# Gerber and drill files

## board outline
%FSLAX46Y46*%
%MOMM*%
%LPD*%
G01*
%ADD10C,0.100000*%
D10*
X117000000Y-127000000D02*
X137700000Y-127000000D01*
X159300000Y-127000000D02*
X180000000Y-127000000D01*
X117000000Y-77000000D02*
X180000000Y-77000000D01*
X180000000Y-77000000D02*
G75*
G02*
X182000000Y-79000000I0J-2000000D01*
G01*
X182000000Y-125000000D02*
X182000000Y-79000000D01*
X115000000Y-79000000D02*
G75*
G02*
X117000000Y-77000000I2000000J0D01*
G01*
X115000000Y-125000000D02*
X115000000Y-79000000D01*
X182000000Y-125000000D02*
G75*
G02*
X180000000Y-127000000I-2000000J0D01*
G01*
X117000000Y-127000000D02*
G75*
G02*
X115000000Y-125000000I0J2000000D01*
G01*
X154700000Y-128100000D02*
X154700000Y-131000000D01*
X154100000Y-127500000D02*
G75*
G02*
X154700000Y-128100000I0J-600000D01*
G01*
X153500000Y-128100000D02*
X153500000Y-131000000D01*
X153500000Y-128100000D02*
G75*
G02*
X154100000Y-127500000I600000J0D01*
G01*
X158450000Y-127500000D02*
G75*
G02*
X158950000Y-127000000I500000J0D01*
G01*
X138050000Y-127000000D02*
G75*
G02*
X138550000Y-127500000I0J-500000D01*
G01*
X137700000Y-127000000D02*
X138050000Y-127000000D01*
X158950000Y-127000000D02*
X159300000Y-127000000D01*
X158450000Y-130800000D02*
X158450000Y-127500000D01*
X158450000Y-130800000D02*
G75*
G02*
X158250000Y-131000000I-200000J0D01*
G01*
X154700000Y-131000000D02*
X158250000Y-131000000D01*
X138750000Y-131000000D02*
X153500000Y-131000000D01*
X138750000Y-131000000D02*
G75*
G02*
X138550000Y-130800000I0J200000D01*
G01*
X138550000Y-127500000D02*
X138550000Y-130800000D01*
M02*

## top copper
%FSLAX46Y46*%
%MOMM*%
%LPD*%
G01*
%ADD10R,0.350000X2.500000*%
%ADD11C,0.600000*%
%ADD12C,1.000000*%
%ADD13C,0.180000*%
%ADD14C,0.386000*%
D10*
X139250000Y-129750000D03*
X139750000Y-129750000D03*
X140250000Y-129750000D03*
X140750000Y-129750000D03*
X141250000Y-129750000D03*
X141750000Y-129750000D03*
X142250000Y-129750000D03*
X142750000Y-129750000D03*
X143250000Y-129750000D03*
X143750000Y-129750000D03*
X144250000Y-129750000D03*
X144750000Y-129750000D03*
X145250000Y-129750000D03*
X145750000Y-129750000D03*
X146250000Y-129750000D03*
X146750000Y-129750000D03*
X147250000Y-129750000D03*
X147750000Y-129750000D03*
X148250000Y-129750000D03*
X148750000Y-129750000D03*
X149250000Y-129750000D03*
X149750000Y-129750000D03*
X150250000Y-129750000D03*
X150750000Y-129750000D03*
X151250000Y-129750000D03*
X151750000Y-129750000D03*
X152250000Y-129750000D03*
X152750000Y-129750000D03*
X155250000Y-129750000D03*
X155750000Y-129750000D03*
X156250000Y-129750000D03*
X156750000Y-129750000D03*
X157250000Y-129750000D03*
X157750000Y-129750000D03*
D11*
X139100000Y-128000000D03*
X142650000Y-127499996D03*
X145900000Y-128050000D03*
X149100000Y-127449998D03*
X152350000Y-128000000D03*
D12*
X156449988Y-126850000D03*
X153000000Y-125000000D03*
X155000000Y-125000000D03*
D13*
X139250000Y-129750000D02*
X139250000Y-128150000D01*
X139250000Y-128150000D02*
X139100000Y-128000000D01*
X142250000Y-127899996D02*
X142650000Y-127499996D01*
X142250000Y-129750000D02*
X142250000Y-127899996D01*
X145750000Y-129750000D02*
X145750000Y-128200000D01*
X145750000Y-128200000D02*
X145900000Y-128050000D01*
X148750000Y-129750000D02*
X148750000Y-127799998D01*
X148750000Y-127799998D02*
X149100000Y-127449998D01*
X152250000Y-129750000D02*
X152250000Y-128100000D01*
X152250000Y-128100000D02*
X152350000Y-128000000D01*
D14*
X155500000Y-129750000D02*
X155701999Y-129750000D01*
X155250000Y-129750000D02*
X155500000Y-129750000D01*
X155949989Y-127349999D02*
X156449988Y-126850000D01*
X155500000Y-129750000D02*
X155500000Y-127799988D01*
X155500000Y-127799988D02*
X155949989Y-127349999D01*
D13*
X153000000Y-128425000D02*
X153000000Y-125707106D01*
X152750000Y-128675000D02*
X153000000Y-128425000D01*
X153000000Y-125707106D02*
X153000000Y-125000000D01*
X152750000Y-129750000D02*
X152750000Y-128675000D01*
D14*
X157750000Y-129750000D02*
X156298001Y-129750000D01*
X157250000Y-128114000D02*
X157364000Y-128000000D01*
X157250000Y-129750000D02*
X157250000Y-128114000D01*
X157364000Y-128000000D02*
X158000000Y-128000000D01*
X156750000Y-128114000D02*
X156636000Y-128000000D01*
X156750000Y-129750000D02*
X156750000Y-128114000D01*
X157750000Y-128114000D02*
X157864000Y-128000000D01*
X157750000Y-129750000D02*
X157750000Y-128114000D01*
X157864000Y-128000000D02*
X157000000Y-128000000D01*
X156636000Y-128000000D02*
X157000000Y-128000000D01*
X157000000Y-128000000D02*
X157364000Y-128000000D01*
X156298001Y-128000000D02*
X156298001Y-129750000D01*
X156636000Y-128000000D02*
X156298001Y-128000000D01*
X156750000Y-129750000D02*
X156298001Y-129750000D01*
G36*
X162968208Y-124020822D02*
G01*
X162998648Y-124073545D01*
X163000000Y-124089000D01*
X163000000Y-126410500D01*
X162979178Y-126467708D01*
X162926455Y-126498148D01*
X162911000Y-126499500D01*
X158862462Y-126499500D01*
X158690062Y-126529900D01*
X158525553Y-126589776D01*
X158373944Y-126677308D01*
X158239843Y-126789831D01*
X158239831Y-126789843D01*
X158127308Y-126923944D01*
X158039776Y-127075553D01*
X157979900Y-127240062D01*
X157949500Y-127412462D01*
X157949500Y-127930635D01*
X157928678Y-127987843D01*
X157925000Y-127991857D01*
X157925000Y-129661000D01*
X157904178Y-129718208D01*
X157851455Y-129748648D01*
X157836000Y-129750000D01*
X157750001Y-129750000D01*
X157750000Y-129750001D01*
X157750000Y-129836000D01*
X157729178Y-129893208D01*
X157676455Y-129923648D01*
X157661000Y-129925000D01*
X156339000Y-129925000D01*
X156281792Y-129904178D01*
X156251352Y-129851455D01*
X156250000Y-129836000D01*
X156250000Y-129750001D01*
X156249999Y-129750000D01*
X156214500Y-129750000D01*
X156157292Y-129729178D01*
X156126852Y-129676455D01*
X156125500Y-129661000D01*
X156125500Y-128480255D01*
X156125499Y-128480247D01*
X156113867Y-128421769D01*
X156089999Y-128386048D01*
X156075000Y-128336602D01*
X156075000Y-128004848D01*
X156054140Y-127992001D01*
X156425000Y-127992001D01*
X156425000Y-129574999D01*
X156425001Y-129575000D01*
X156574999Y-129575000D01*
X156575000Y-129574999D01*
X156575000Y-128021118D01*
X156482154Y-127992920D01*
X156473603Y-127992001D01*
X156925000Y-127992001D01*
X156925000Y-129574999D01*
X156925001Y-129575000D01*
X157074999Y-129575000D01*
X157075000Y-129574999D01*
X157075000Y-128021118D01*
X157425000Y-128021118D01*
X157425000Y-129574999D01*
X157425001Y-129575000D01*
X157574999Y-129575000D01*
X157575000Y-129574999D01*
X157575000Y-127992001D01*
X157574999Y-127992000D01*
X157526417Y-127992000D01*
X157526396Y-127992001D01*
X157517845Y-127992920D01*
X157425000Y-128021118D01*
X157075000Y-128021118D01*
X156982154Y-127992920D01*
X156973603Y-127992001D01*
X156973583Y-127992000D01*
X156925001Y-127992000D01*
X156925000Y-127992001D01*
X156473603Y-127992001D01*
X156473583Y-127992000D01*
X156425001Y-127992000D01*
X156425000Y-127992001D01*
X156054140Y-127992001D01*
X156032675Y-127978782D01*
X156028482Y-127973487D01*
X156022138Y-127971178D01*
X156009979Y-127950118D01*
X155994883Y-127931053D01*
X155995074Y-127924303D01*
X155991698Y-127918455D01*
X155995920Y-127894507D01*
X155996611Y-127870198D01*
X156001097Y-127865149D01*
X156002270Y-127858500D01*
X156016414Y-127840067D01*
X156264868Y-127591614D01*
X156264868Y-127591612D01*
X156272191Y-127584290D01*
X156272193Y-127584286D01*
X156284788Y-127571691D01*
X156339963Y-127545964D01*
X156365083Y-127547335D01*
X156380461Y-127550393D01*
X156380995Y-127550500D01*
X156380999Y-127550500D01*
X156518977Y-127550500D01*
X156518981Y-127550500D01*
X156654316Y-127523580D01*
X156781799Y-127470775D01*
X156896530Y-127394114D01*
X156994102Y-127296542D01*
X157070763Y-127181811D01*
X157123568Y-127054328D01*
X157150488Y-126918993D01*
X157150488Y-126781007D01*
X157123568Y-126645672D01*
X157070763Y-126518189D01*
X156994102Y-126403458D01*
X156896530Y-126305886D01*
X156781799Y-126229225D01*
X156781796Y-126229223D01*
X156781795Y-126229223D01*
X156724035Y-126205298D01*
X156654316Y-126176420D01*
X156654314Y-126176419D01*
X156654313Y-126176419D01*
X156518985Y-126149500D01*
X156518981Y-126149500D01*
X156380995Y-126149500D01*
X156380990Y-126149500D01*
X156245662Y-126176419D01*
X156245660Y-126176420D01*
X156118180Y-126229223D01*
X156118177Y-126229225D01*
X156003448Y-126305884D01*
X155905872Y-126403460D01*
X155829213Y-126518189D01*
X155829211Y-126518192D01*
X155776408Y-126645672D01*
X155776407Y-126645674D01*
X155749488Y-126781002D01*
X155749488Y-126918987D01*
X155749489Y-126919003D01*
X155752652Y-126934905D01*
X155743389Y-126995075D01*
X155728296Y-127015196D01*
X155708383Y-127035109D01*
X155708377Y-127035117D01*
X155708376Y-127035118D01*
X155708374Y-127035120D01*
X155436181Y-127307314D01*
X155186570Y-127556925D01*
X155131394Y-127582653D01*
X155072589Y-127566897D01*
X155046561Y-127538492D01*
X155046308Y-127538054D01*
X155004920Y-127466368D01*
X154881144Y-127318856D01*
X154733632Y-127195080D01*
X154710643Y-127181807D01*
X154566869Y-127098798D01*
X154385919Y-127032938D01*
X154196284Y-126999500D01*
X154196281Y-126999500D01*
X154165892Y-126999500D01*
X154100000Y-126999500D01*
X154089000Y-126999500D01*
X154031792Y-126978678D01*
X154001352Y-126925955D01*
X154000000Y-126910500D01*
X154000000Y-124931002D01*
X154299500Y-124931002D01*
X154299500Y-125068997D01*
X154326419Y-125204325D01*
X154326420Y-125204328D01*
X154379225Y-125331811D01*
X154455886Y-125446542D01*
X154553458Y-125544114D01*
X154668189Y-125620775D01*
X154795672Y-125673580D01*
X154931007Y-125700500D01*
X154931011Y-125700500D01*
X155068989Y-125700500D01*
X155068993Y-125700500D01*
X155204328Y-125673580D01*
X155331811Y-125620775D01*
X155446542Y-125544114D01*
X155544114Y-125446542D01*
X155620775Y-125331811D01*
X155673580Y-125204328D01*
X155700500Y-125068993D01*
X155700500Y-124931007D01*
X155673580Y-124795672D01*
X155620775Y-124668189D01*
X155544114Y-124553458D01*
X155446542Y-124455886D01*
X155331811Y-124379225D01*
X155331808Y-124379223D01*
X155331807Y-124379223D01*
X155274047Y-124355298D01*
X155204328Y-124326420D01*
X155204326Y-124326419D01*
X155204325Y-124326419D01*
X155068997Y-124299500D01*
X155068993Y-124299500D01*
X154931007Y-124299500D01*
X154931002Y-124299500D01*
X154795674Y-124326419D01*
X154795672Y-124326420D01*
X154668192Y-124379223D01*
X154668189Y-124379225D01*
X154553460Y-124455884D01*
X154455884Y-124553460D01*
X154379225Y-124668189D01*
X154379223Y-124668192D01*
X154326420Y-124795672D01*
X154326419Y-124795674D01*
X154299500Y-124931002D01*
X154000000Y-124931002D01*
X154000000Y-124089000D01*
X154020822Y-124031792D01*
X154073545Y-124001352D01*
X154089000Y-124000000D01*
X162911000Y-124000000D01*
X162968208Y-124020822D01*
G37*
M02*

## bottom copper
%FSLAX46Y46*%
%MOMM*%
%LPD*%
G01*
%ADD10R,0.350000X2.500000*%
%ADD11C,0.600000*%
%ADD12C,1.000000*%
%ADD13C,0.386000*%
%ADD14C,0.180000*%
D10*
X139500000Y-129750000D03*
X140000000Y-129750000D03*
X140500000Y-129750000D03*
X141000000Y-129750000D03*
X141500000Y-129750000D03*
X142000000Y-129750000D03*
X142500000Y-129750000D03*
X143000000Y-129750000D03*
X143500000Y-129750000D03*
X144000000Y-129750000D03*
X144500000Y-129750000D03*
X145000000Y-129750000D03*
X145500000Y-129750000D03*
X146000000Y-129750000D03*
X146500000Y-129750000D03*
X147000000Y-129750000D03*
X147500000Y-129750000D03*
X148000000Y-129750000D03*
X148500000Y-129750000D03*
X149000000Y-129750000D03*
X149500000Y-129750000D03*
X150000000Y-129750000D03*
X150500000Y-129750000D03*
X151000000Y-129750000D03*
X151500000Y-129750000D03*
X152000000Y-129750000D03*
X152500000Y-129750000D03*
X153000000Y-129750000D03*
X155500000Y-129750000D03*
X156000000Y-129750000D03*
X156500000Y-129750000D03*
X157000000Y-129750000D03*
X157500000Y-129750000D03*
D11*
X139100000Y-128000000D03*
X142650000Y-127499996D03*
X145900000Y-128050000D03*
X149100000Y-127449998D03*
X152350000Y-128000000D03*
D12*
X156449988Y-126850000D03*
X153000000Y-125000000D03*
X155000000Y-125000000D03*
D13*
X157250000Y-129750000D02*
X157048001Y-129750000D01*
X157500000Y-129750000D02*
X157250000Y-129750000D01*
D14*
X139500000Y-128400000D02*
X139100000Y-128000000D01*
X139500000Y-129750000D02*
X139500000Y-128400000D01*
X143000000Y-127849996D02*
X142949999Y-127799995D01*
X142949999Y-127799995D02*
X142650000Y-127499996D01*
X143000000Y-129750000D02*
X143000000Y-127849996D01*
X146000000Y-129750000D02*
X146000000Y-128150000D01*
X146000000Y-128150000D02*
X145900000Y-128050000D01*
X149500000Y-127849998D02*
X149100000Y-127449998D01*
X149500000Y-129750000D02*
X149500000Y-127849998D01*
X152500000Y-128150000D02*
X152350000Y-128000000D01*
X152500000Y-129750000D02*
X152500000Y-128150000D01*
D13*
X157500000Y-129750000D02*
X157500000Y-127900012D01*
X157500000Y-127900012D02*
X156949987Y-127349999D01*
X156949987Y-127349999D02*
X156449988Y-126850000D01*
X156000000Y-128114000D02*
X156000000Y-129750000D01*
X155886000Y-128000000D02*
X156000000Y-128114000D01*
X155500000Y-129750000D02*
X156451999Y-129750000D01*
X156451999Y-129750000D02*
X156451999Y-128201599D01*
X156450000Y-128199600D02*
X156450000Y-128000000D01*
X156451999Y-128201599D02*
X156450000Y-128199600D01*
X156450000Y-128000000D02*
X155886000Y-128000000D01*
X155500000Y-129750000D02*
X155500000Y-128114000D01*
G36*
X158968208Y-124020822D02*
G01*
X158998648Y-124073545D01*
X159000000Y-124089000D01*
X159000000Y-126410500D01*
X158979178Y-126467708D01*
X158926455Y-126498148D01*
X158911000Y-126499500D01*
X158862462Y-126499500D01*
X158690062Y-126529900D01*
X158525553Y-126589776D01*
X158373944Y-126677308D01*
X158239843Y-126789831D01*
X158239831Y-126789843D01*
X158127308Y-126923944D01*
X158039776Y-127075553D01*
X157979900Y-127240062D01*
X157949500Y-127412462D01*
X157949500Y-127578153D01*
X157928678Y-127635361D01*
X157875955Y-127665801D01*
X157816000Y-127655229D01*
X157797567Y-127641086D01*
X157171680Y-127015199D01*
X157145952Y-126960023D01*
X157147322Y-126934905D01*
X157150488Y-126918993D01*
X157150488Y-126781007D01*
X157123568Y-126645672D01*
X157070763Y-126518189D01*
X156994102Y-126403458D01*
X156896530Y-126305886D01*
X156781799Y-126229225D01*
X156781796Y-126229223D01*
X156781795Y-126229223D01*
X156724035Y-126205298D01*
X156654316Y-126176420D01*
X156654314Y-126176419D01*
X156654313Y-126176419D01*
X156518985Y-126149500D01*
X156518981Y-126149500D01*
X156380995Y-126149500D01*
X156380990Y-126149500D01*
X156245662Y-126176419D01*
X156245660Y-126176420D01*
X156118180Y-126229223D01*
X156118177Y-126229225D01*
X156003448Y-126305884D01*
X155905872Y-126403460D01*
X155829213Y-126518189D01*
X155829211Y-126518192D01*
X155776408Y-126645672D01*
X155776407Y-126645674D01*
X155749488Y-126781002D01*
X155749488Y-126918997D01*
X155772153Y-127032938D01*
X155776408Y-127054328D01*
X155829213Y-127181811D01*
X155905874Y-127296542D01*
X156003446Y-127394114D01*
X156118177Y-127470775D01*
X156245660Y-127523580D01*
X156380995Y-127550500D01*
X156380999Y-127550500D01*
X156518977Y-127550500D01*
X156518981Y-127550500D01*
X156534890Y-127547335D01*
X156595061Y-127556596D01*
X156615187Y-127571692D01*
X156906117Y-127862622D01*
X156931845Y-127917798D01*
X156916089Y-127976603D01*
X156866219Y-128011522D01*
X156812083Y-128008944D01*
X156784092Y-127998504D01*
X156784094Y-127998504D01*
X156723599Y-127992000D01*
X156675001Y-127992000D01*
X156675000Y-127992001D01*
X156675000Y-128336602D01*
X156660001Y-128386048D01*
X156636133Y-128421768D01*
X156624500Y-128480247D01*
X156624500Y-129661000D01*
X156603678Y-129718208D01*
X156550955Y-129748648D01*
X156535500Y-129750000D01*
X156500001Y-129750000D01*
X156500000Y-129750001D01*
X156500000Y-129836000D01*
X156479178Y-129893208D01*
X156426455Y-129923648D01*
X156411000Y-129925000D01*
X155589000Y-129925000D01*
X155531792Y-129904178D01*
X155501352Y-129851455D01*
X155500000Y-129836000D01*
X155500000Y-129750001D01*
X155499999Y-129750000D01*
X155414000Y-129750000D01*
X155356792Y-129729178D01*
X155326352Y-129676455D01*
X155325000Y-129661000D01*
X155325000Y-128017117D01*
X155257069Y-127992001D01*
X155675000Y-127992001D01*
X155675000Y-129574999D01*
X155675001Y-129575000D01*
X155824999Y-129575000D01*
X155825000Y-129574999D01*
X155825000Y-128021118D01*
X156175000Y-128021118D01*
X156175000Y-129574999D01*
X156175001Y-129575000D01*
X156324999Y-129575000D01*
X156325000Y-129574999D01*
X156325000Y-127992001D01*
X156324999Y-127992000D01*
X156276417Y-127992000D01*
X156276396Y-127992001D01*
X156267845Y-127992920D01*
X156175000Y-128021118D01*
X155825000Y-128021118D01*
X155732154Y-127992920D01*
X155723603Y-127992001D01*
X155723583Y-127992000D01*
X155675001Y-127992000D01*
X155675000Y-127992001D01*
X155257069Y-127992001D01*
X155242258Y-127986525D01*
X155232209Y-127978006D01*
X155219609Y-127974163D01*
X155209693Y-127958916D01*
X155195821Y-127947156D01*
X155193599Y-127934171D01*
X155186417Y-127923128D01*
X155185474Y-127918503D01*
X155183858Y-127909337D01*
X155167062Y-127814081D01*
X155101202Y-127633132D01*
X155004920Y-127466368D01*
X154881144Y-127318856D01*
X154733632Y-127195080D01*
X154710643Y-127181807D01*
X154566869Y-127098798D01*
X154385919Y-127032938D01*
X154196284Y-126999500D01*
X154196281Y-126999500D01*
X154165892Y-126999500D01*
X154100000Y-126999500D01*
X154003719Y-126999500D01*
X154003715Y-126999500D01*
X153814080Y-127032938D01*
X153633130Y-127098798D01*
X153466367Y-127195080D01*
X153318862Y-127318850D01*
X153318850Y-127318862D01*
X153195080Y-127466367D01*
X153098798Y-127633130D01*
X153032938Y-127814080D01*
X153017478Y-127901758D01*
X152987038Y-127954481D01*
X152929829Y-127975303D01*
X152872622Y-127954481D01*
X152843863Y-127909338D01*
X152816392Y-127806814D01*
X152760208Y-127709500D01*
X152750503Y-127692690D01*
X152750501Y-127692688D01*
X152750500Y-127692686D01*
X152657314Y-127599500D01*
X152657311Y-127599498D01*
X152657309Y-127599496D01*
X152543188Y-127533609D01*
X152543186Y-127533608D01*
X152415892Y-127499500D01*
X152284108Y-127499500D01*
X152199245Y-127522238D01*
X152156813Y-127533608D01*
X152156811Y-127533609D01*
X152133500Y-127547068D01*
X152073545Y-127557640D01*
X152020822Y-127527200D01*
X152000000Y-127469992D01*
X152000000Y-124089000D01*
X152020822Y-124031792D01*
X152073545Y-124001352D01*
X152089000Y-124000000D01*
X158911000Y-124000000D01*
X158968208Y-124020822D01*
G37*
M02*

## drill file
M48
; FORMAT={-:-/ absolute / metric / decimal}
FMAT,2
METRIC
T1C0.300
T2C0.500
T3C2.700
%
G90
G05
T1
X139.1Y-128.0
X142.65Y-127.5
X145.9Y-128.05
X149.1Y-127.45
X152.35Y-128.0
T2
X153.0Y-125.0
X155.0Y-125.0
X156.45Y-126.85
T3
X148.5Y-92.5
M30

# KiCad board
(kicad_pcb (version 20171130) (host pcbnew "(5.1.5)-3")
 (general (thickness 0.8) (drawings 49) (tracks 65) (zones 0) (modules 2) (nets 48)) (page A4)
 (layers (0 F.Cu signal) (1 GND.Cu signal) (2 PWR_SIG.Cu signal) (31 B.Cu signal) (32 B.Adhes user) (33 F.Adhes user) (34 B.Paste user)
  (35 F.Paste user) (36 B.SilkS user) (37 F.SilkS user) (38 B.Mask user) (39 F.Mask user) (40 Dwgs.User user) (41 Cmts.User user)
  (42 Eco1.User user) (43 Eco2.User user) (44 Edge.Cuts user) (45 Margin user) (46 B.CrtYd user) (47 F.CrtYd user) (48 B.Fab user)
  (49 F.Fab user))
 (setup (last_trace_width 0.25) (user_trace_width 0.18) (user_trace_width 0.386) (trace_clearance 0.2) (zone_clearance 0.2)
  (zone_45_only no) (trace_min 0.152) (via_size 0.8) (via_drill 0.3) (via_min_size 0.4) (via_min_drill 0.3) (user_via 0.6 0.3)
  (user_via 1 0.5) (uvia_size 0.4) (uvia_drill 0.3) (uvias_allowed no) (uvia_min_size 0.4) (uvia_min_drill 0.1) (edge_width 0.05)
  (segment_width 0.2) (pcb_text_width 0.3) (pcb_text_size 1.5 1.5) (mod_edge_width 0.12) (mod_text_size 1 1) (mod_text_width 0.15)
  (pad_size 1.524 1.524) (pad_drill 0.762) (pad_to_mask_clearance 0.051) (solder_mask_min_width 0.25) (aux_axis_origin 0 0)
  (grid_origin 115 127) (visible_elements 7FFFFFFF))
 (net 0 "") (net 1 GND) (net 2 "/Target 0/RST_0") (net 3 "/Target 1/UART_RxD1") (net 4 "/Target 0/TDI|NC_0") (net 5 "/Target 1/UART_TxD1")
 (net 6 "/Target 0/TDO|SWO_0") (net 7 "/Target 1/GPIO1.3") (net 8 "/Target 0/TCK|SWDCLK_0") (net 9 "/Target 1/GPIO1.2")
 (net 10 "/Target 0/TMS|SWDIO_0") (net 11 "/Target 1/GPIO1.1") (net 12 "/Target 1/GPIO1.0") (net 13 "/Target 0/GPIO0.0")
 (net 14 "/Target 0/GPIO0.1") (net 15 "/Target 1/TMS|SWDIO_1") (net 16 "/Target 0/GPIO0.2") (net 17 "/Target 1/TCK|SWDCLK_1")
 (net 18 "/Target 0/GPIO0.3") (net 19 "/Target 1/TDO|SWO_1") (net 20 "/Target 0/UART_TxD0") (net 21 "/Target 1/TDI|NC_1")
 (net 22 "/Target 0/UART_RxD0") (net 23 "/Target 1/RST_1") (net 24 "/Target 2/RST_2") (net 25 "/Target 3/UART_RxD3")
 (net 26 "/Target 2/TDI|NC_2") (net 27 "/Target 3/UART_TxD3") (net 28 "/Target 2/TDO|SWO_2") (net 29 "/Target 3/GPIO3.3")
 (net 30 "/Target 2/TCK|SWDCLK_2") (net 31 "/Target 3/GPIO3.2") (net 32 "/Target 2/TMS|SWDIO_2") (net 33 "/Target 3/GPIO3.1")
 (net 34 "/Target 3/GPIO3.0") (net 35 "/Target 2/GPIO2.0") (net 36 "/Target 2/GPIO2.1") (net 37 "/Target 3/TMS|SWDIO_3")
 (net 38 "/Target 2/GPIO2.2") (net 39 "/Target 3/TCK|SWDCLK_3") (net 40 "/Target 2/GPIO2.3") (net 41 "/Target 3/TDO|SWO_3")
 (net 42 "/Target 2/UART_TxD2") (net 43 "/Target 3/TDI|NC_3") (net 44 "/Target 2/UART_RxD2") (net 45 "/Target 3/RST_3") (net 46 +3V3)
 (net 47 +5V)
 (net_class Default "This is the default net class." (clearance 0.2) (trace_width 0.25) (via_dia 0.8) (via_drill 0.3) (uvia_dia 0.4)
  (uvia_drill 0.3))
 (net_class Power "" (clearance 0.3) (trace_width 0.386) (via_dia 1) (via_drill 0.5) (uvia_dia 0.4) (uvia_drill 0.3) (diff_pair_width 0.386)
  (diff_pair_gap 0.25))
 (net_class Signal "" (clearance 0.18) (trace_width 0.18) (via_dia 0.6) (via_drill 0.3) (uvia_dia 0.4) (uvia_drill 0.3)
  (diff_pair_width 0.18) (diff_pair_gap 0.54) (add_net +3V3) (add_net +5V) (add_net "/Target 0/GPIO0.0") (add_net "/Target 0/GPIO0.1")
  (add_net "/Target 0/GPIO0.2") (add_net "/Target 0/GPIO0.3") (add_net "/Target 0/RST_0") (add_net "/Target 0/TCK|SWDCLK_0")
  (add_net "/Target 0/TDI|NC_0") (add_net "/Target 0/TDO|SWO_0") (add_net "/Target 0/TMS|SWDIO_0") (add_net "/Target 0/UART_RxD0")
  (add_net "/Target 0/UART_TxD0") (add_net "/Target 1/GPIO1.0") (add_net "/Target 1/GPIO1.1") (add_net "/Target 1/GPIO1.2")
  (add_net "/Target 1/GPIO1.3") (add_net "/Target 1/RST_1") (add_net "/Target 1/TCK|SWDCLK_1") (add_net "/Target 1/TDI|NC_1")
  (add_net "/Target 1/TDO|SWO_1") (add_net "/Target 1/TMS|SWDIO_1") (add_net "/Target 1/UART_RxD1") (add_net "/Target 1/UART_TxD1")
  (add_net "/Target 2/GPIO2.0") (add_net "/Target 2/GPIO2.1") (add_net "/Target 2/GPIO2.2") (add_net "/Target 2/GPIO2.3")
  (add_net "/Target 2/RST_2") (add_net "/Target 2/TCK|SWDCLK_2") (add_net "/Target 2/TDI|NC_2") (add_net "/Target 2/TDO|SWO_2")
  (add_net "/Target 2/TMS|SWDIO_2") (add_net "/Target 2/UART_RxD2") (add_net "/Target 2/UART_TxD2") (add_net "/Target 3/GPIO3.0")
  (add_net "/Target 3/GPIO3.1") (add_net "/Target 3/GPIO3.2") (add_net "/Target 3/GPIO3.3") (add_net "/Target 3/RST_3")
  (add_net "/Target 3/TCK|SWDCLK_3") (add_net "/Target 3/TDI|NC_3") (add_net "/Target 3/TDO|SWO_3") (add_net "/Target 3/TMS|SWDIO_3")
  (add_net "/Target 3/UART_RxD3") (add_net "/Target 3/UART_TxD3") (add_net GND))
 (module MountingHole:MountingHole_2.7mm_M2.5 (layer F.Cu) (at 148.5 92.5)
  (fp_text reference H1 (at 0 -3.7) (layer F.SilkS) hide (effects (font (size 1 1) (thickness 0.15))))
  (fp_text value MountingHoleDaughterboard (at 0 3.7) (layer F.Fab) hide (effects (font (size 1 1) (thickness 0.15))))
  (pad 1 np_thru_hole circle (at 0 0) (size 2.7 2.7) (drill 2.7) (layers *.Cu *.Mask)))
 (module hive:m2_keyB (layer F.Cu) (at 148.5 131)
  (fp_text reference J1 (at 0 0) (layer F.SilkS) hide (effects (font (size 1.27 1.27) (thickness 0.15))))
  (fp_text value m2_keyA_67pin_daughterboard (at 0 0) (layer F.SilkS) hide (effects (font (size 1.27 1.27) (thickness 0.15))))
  (fp_line (start 6.2 -2.9) (end 6.2 0) (layer Edge.Cuts) (width 0.1))
  (fp_arc (start 5.6 -2.9) (end 5.6 -3.5) (angle 90) (layer Edge.Cuts) (width 0.1))
  (fp_line (start 5 -2.9) (end 5 0) (layer Edge.Cuts) (width 0.1))
  (fp_arc (start 5.6 -2.9) (end 5.6 -3.5) (angle -90) (layer Edge.Cuts) (width 0.1))
  (fp_arc (start 10.45 -3.5) (end 9.95 -3.5) (angle 90) (layer Edge.Cuts) (width 0.1))
  (fp_arc (start -10.45 -3.5) (end -10.45 -4) (angle 90) (layer Edge.Cuts) (width 0.1))
  (fp_line (start -10.8 -4) (end -10.45 -4) (layer Edge.Cuts) (width 0.1))
  (fp_line (start 10.45 -4) (end 10.8 -4) (layer Edge.Cuts) (width 0.1))
  (fp_line (start 9.95 -0.2) (end 9.95 -3.5) (layer Edge.Cuts) (width 0.1))
  (fp_arc (start 9.75 -0.2) (end 9.75 0) (angle -90) (layer Edge.Cuts) (width 0.1))
  (fp_line (start 6.2 0) (end 9.75 0) (layer Edge.Cuts) (width 0.1))
  (fp_line (start -9.75 0) (end 5 0) (layer Edge.Cuts) (width 0.1))
  (fp_arc (start -9.75 -0.2) (end -9.95 -0.2) (angle -90) (layer Edge.Cuts) (width 0.1))
  (fp_line (start -9.95 -3.5) (end -9.95 -0.2) (layer Edge.Cuts) (width 0.1))
  (pad 75 smd rect (at -9.25 -1.25) (size 0.35 2.5) (layers F.Cu F.Paste F.Mask) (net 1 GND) (solder_mask_margin 0.1016))
  (pad 74 smd rect (at -9 -1.25) (size 0.35 2.5) (layers B.Cu B.Paste B.Mask) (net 1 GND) (solder_mask_margin 0.1016))
  (pad 73 smd rect (at -8.75 -1.25) (size 0.35 2.5) (layers F.Cu F.Paste F.Mask) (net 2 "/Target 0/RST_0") (solder_mask_margin 0.1016))
  (pad 72 smd rect (at -8.5 -1.25) (size 0.35 2.5) (layers B.Cu B.Paste B.Mask) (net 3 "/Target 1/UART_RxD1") (solder_mask_margin 0.1016))
  (pad 71 smd rect (at -8.25 -1.25) (size 0.35 2.5) (layers F.Cu F.Paste F.Mask) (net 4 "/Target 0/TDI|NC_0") (solder_mask_margin 0.1016))
  (pad 70 smd rect (at -8 -1.25) (size 0.35 2.5) (layers B.Cu B.Paste B.Mask) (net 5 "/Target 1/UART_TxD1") (solder_mask_margin 0.1016))
  (pad 69 smd rect (at -7.75 -1.25) (size 0.35 2.5) (layers F.Cu F.Paste F.Mask) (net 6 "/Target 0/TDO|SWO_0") (solder_mask_margin 0.1016))
  (pad 68 smd rect (at -7.5 -1.25) (size 0.35 2.5) (layers B.Cu B.Paste B.Mask) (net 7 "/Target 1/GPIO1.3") (solder_mask_margin 0.1016))
  (pad 67 smd rect (at -7.25 -1.25) (size 0.35 2.5) (layers F.Cu F.Paste F.Mask) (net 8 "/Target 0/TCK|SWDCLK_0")
   (solder_mask_margin 0.1016))
  (pad 66 smd rect (at -7 -1.25) (size 0.35 2.5) (layers B.Cu B.Paste B.Mask) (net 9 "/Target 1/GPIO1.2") (solder_mask_margin 0.1016))
  (pad 65 smd rect (at -6.75 -1.25) (size 0.35 2.5) (layers F.Cu F.Paste F.Mask) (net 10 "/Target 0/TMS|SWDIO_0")
   (solder_mask_margin 0.1016))
  (pad 64 smd rect (at -6.5 -1.25) (size 0.35 2.5) (layers B.Cu B.Paste B.Mask) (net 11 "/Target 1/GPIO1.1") (solder_mask_margin 0.1016))
  (pad 63 smd rect (at -6.25 -1.25) (size 0.35 2.5) (layers F.Cu F.Paste F.Mask) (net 1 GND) (solder_mask_margin 0.1016))
  (pad 62 smd rect (at -6 -1.25) (size 0.35 2.5) (layers B.Cu B.Paste B.Mask) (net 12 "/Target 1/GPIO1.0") (solder_mask_margin 0.1016))
  (pad 61 smd rect (at -5.75 -1.25) (size 0.35 2.5) (layers F.Cu F.Paste F.Mask) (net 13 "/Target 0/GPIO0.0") (solder_mask_margin 0.1016))
  (pad 60 smd rect (at -5.5 -1.25) (size 0.35 2.5) (layers B.Cu B.Paste B.Mask) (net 1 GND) (solder_mask_margin 0.1016))
  (pad 59 smd rect (at -5.25 -1.25) (size 0.35 2.5) (layers F.Cu F.Paste F.Mask) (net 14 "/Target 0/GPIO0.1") (solder_mask_margin 0.1016))
  (pad 58 smd rect (at -5 -1.25) (size 0.35 2.5) (layers B.Cu B.Paste B.Mask) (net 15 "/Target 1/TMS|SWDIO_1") (solder_mask_margin 0.1016))
  (pad 57 smd rect (at -4.75 -1.25) (size 0.35 2.5) (layers F.Cu F.Paste F.Mask) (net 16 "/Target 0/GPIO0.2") (solder_mask_margin 0.1016))
  (pad 56 smd rect (at -4.5 -1.25) (size 0.35 2.5) (layers B.Cu B.Paste B.Mask) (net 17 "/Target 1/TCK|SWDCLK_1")
   (solder_mask_margin 0.1016))
  (pad 55 smd rect (at -4.25 -1.25) (size 0.35 2.5) (layers F.Cu F.Paste F.Mask) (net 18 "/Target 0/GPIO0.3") (solder_mask_margin 0.1016))
  (pad 54 smd rect (at -4 -1.25) (size 0.35 2.5) (layers B.Cu B.Paste B.Mask) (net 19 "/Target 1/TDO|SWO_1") (solder_mask_margin 0.1016))
  (pad 53 smd rect (at -3.75 -1.25) (size 0.35 2.5) (layers F.Cu F.Paste F.Mask) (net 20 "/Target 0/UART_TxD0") (solder_mask_margin 0.1016))
  (pad 52 smd rect (at -3.5 -1.25) (size 0.35 2.5) (layers B.Cu B.Paste B.Mask) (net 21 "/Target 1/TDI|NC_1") (solder_mask_margin 0.1016))
  (pad 51 smd rect (at -3.25 -1.25) (size 0.35 2.5) (layers F.Cu F.Paste F.Mask) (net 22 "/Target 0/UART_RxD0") (solder_mask_margin 0.1016))
  (pad 50 smd rect (at -3 -1.25) (size 0.35 2.5) (layers B.Cu B.Paste B.Mask) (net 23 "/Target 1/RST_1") (solder_mask_margin 0.1016))
  (pad 49 smd rect (at -2.75 -1.25) (size 0.35 2.5) (layers F.Cu F.Paste F.Mask) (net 1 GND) (solder_mask_margin 0.1016))
  (pad 48 smd rect (at -2.5 -1.25) (size 0.35 2.5) (layers B.Cu B.Paste B.Mask) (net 1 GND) (solder_mask_margin 0.1016))
  (pad 47 smd rect (at -2.25 -1.25) (size 0.35 2.5) (layers F.Cu F.Paste F.Mask) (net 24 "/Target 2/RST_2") (solder_mask_margin 0.1016))
  (pad 46 smd rect (at -2 -1.25) (size 0.35 2.5) (layers B.Cu B.Paste B.Mask) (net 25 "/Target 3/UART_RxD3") (solder_mask_margin 0.1016))
  (pad 45 smd rect (at -1.75 -1.25) (size 0.35 2.5) (layers F.Cu F.Paste F.Mask) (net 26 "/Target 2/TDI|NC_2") (solder_mask_margin 0.1016))
  (pad 44 smd rect (at -1.5 -1.25) (size 0.35 2.5) (layers B.Cu B.Paste B.Mask) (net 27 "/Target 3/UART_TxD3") (solder_mask_margin 0.1016))
  (pad 43 smd rect (at -1.25 -1.25) (size 0.35 2.5) (layers F.Cu F.Paste F.Mask) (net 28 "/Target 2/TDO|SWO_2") (solder_mask_margin 0.1016))
  (pad 42 smd rect (at -1 -1.25) (size 0.35 2.5) (layers B.Cu B.Paste B.Mask) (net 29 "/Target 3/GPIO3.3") (solder_mask_margin 0.1016))
  (pad 41 smd rect (at -0.75 -1.25) (size 0.35 2.5) (layers F.Cu F.Paste F.Mask) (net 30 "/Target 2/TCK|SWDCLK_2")
   (solder_mask_margin 0.1016))
  (pad 40 smd rect (at -0.5 -1.25) (size 0.35 2.5) (layers B.Cu B.Paste B.Mask) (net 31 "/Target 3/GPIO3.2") (solder_mask_margin 0.1016))
  (pad 39 smd rect (at -0.25 -1.25) (size 0.35 2.5) (layers F.Cu F.Paste F.Mask) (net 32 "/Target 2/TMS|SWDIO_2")
   (solder_mask_margin 0.1016))
  (pad 38 smd rect (at 0 -1.25) (size 0.35 2.5) (layers B.Cu B.Paste B.Mask) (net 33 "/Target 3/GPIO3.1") (solder_mask_margin 0.1016))
  (pad 37 smd rect (at 0.25 -1.25) (size 0.35 2.5) (layers F.Cu F.Paste F.Mask) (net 1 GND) (solder_mask_margin 0.1016))
  (pad 36 smd rect (at 0.5 -1.25) (size 0.35 2.5) (layers B.Cu B.Paste B.Mask) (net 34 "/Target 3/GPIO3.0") (solder_mask_margin 0.1016))
  (pad 35 smd rect (at 0.75 -1.25) (size 0.35 2.5) (layers F.Cu F.Paste F.Mask) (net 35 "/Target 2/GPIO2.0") (solder_mask_margin 0.1016))
  (pad 34 smd rect (at 1 -1.25) (size 0.35 2.5) (layers B.Cu B.Paste B.Mask) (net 1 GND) (solder_mask_margin 0.1016))
  (pad 33 smd rect (at 1.25 -1.25) (size 0.35 2.5) (layers F.Cu F.Paste F.Mask) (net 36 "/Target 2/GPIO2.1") (solder_mask_margin 0.1016))
  (pad 32 smd rect (at 1.5 -1.25) (size 0.35 2.5) (layers B.Cu B.Paste B.Mask) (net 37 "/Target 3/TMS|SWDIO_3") (solder_mask_margin 0.1016))
  (pad 31 smd rect (at 1.75 -1.25) (size 0.35 2.5) (layers F.Cu F.Paste F.Mask) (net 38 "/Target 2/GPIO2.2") (solder_mask_margin 0.1016))
  (pad 30 smd rect (at 2 -1.25) (size 0.35 2.5) (layers B.Cu B.Paste B.Mask) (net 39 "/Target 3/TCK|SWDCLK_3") (solder_mask_margin 0.1016))
  (pad 29 smd rect (at 2.25 -1.25) (size 0.35 2.5) (layers F.Cu F.Paste F.Mask) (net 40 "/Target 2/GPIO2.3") (solder_mask_margin 0.1016))
  (pad 28 smd rect (at 2.5 -1.25) (size 0.35 2.5) (layers B.Cu B.Paste B.Mask) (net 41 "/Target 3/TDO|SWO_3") (solder_mask_margin 0.1016))
  (pad 27 smd rect (at 2.75 -1.25) (size 0.35 2.5) (layers F.Cu F.Paste F.Mask) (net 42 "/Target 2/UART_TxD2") (solder_mask_margin 0.1016))
  (pad 26 smd rect (at 3 -1.25) (size 0.35 2.5) (layers B.Cu B.Paste B.Mask) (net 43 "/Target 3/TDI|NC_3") (solder_mask_margin 0.1016))
  (pad 25 smd rect (at 3.25 -1.25) (size 0.35 2.5) (layers F.Cu F.Paste F.Mask) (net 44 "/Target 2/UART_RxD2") (solder_mask_margin 0.1016))
  (pad 24 smd rect (at 3.5 -1.25) (size 0.35 2.5) (layers B.Cu B.Paste B.Mask) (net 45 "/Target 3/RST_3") (solder_mask_margin 0.1016))
  (pad 23 smd rect (at 3.75 -1.25) (size 0.35 2.5) (layers F.Cu F.Paste F.Mask) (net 1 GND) (solder_mask_margin 0.1016))
  (pad 22 smd rect (at 4 -1.25) (size 0.35 2.5) (layers B.Cu B.Paste B.Mask) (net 1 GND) (solder_mask_margin 0.1016))
  (pad 21 smd rect (at 4.25 -1.25) (size 0.35 2.5) (layers F.Cu F.Paste F.Mask) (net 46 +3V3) (solder_mask_margin 0.1016))
  (pad 20 smd rect (at 4.5 -1.25) (size 0.35 2.5) (layers B.Cu B.Paste B.Mask) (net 46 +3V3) (solder_mask_margin 0.1016))
  (pad 11 smd rect (at 6.75 -1.25) (size 0.35 2.5) (layers F.Cu F.Paste F.Mask) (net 1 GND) (solder_mask_margin 0.1016))
  (pad 10 smd rect (at 7 -1.25) (size 0.35 2.5) (layers B.Cu B.Paste B.Mask) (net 46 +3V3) (solder_mask_margin 0.1016))
  (pad 9 smd rect (at 7.25 -1.25) (size 0.35 2.5) (layers F.Cu F.Paste F.Mask) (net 1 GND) (solder_mask_margin 0.1016))
  (pad 8 smd rect (at 7.5 -1.25) (size 0.35 2.5) (layers B.Cu B.Paste B.Mask) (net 46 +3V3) (solder_mask_margin 0.1016))
  (pad 7 smd rect (at 7.75 -1.25) (size 0.35 2.5) (layers F.Cu F.Paste F.Mask) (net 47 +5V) (solder_mask_margin 0.1016))
  (pad 6 smd rect (at 8 -1.25) (size 0.35 2.5) (layers B.Cu B.Paste B.Mask) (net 46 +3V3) (solder_mask_margin 0.1016))
  (pad 5 smd rect (at 8.25 -1.25) (size 0.35 2.5) (layers F.Cu F.Paste F.Mask) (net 47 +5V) (solder_mask_margin 0.1016))
  (pad 4 smd rect (at 8.5 -1.25) (size 0.35 2.5) (layers B.Cu B.Paste B.Mask) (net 1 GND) (solder_mask_margin 0.1016))
  (pad 3 smd rect (at 8.75 -1.25) (size 0.35 2.5) (layers F.Cu F.Paste F.Mask) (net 47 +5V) (solder_mask_margin 0.1016))
  (pad 2 smd rect (at 9 -1.25) (size 0.35 2.5) (layers B.Cu B.Paste B.Mask) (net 1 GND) (solder_mask_margin 0.1016))
  (pad 1 smd rect (at 9.25 -1.25) (size 0.35 2.5) (layers F.Cu F.Paste F.Mask) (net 47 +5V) (solder_mask_margin 0.1016)))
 (gr_line (start 117 127) (end 137.7 127) (layer Edge.Cuts) (width 0.1))
 (gr_line (start 159.3 127) (end 180 127) (layer Edge.Cuts) (width 0.1))
 (gr_line (start 117 77) (end 180 77) (layer Edge.Cuts) (width 0.1))
 (gr_arc (start 180 79) (end 182 79) (angle -90) (layer Edge.Cuts) (width 0.1))
 (gr_line (start 182 125) (end 182 79) (layer Edge.Cuts) (width 0.1))
 (gr_arc (start 117 79) (end 117 77) (angle -90) (layer Edge.Cuts) (width 0.1))
 (gr_line (start 115 125) (end 115 79) (layer Edge.Cuts) (width 0.1))
 (gr_arc (start 180 125) (end 180 127) (angle -90) (layer Edge.Cuts) (width 0.1))
 (gr_arc (start 117 125) (end 115 125) (angle -90) (layer Edge.Cuts) (width 0.1))
 (segment (start 157.25 129.75) (end 157.048001 129.75) (width 0.386) (layer B.Cu) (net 1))
 (segment (start 157.5 129.75) (end 157.25 129.75) (width 0.386) (layer B.Cu) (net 1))
 (via (at 139.1 128) (size 0.6) (drill 0.3) (layers F.Cu B.Cu) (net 1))
 (segment (start 139.25 129.75) (end 139.25 128.15) (width 0.18) (layer F.Cu) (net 1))
 (segment (start 139.25 128.15) (end 139.1 128) (width 0.18) (layer F.Cu) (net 1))
 (segment (start 139.5 128.4) (end 139.1 128) (width 0.18) (layer B.Cu) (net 1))
 (segment (start 139.5 129.75) (end 139.5 128.4) (width 0.18) (layer B.Cu) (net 1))
 (segment (start 143 127.849996) (end 142.949999 127.799995) (width 0.18) (layer B.Cu) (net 1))
 (segment (start 142.949999 127.799995) (end 142.65 127.499996) (width 0.18) (layer B.Cu) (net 1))
 (via (at 142.65 127.499996) (size 0.6) (drill 0.3) (layers F.Cu B.Cu) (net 1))
 (segment (start 143 129.75) (end 143 127.849996) (width 0.18) (layer B.Cu) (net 1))
 (segment (start 142.25 127.899996) (end 142.65 127.499996) (width 0.18) (layer F.Cu) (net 1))
 (segment (start 142.25 129.75) (end 142.25 127.899996) (width 0.18) (layer F.Cu) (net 1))
 (via (at 145.9 128.05) (size 0.6) (drill 0.3) (layers F.Cu B.Cu) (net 1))
 (segment (start 146 129.75) (end 146 128.15) (width 0.18) (layer B.Cu) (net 1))
 (segment (start 145.75 129.75) (end 145.75 128.2) (width 0.18) (layer F.Cu) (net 1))
 (segment (start 146 128.15) (end 145.9 128.05) (width 0.18) (layer B.Cu) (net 1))
 (segment (start 145.75 128.2) (end 145.9 128.05) (width 0.18) (layer F.Cu) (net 1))
 (via (at 149.1 127.449998) (size 0.6) (drill 0.3) (layers F.Cu B.Cu) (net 1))
 (segment (start 149.5 127.849998) (end 149.1 127.449998) (width 0.18) (layer B.Cu) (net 1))
 (segment (start 148.75 129.75) (end 148.75 127.799998) (width 0.18) (layer F.Cu) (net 1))
 (segment (start 149.5 129.75) (end 149.5 127.849998) (width 0.18) (layer B.Cu) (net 1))
 (segment (start 148.75 127.799998) (end 149.1 127.449998) (width 0.18) (layer F.Cu) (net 1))
 (segment (start 152.25 129.75) (end 152.25 128.1) (width 0.18) (layer F.Cu) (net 1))
 (segment (start 152.5 128.15) (end 152.35 128) (width 0.18) (layer B.Cu) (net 1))
 (segment (start 152.5 129.75) (end 152.5 128.15) (width 0.18) (layer B.Cu) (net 1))
 (via (at 152.35 128) (size 0.6) (drill 0.3) (layers F.Cu B.Cu) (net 1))
 (segment (start 152.25 128.1) (end 152.35 128) (width 0.18) (layer F.Cu) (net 1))
 (segment (start 155.5 129.75) (end 155.701999 129.75) (width 0.386) (layer F.Cu) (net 1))
 (segment (start 155.25 129.75) (end 155.5 129.75) (width 0.386) (layer F.Cu) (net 1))
 (via (at 156.449988 126.85) (size 1) (drill 0.5) (layers F.Cu B.Cu) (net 1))
 (segment (start 157.5 129.75) (end 157.5 127.900012) (width 0.386) (layer B.Cu) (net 1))
 (segment (start 157.5 127.900012) (end 156.949987 127.349999) (width 0.386) (layer B.Cu) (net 1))
 (segment (start 156.949987 127.349999) (end 156.449988 126.85) (width 0.386) (layer B.Cu) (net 1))
 (segment (start 155.949989 127.349999) (end 156.449988 126.85) (width 0.386) (layer F.Cu) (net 1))
 (segment (start 155.5 129.75) (end 155.5 127.799988) (width 0.386) (layer F.Cu) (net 1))
 (segment (start 155.5 127.799988) (end 155.949989 127.349999) (width 0.386) (layer F.Cu) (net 1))
 (via (at 153 125) (size 1) (drill 0.5) (layers F.Cu B.Cu) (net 46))
 (segment (start 156 128.114) (end 156 129.75) (width 0.386) (layer B.Cu) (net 46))
 (segment (start 155.886 128) (end 156 128.114) (width 0.386) (layer B.Cu) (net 46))
 (segment (start 155.5 129.75) (end 156.451999 129.75) (width 0.386) (layer B.Cu) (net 46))
 (segment (start 156.451999 129.75) (end 156.451999 128.201599) (width 0.386) (layer B.Cu) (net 46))
 (segment (start 156.45 128.1996) (end 156.45 128) (width 0.386) (layer B.Cu) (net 46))
 (segment (start 156.451999 128.201599) (end 156.45 128.1996) (width 0.386) (layer B.Cu) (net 46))
 (segment (start 156.45 128) (end 155.886 128) (width 0.386) (layer B.Cu) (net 46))
 (segment (start 155.5 129.75) (end 155.5 128.114) (width 0.386) (layer B.Cu) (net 46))
 (via (at 155 125) (size 1) (drill 0.5) (layers F.Cu B.Cu) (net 46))
 (segment (start 153 128.425) (end 153 125.707106) (width 0.18) (layer F.Cu) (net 46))
 (segment (start 152.75 128.675) (end 153 128.425) (width 0.18) (layer F.Cu) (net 46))
 (segment (start 153 125.707106) (end 153 125) (width 0.18) (layer F.Cu) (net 46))
 (segment (start 152.75 129.75) (end 152.75 128.675) (width 0.18) (layer F.Cu) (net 46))
 (segment (start 157.75 129.75) (end 156.298001 129.75) (width 0.386) (layer F.Cu) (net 47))
 (segment (start 157.25 128.114) (end 157.364 128) (width 0.386) (layer F.Cu) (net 47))
 (segment (start 157.25 129.75) (end 157.25 128.114) (width 0.386) (layer F.Cu) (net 47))
 (segment (start 157.364 128) (end 158 128) (width 0.386) (layer F.Cu) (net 47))
 (segment (start 156.75 128.114) (end 156.636 128) (width 0.386) (layer F.Cu) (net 47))
 (segment (start 156.75 129.75) (end 156.75 128.114) (width 0.386) (layer F.Cu) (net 47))
 (segment (start 157.75 128.114) (end 157.864 128) (width 0.386) (layer F.Cu) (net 47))
 (segment (start 157.75 129.75) (end 157.75 128.114) (width 0.386) (layer F.Cu) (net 47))
 (segment (start 157.864 128) (end 157 128) (width 0.386) (layer F.Cu) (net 47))
 (segment (start 156.636 128) (end 157 128) (width 0.386) (layer F.Cu) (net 47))
 (segment (start 157 128) (end 157.364 128) (width 0.386) (layer F.Cu) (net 47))
 (segment (start 156.298001 128) (end 156.298001 129.75) (width 0.386) (layer F.Cu) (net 47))
 (segment (start 156.636 128) (end 156.298001 128) (width 0.386) (layer F.Cu) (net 47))
 (segment (start 156.75 129.75) (end 156.298001 129.75) (width 0.386) (layer F.Cu) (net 47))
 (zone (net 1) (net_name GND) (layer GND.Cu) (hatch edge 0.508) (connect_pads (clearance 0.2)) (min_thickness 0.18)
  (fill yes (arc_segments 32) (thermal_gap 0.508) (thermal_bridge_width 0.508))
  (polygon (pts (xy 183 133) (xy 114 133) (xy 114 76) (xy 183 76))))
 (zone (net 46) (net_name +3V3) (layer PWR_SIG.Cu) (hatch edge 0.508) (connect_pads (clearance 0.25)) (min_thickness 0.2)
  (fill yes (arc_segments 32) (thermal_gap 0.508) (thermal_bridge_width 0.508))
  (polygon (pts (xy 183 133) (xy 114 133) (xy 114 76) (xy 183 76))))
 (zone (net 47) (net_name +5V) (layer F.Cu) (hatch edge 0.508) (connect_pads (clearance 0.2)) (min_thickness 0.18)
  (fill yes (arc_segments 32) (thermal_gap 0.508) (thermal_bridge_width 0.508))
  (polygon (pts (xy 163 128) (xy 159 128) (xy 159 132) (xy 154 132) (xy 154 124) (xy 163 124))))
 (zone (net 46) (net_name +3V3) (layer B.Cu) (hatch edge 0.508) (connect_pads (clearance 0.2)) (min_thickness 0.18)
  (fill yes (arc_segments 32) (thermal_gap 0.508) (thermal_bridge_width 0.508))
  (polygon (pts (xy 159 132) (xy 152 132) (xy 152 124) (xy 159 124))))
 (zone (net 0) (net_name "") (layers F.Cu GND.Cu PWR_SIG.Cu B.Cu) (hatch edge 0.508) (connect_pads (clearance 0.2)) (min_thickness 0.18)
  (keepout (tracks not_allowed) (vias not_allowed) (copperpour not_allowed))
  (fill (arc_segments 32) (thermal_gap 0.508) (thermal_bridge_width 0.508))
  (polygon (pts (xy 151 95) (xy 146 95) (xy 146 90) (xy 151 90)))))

